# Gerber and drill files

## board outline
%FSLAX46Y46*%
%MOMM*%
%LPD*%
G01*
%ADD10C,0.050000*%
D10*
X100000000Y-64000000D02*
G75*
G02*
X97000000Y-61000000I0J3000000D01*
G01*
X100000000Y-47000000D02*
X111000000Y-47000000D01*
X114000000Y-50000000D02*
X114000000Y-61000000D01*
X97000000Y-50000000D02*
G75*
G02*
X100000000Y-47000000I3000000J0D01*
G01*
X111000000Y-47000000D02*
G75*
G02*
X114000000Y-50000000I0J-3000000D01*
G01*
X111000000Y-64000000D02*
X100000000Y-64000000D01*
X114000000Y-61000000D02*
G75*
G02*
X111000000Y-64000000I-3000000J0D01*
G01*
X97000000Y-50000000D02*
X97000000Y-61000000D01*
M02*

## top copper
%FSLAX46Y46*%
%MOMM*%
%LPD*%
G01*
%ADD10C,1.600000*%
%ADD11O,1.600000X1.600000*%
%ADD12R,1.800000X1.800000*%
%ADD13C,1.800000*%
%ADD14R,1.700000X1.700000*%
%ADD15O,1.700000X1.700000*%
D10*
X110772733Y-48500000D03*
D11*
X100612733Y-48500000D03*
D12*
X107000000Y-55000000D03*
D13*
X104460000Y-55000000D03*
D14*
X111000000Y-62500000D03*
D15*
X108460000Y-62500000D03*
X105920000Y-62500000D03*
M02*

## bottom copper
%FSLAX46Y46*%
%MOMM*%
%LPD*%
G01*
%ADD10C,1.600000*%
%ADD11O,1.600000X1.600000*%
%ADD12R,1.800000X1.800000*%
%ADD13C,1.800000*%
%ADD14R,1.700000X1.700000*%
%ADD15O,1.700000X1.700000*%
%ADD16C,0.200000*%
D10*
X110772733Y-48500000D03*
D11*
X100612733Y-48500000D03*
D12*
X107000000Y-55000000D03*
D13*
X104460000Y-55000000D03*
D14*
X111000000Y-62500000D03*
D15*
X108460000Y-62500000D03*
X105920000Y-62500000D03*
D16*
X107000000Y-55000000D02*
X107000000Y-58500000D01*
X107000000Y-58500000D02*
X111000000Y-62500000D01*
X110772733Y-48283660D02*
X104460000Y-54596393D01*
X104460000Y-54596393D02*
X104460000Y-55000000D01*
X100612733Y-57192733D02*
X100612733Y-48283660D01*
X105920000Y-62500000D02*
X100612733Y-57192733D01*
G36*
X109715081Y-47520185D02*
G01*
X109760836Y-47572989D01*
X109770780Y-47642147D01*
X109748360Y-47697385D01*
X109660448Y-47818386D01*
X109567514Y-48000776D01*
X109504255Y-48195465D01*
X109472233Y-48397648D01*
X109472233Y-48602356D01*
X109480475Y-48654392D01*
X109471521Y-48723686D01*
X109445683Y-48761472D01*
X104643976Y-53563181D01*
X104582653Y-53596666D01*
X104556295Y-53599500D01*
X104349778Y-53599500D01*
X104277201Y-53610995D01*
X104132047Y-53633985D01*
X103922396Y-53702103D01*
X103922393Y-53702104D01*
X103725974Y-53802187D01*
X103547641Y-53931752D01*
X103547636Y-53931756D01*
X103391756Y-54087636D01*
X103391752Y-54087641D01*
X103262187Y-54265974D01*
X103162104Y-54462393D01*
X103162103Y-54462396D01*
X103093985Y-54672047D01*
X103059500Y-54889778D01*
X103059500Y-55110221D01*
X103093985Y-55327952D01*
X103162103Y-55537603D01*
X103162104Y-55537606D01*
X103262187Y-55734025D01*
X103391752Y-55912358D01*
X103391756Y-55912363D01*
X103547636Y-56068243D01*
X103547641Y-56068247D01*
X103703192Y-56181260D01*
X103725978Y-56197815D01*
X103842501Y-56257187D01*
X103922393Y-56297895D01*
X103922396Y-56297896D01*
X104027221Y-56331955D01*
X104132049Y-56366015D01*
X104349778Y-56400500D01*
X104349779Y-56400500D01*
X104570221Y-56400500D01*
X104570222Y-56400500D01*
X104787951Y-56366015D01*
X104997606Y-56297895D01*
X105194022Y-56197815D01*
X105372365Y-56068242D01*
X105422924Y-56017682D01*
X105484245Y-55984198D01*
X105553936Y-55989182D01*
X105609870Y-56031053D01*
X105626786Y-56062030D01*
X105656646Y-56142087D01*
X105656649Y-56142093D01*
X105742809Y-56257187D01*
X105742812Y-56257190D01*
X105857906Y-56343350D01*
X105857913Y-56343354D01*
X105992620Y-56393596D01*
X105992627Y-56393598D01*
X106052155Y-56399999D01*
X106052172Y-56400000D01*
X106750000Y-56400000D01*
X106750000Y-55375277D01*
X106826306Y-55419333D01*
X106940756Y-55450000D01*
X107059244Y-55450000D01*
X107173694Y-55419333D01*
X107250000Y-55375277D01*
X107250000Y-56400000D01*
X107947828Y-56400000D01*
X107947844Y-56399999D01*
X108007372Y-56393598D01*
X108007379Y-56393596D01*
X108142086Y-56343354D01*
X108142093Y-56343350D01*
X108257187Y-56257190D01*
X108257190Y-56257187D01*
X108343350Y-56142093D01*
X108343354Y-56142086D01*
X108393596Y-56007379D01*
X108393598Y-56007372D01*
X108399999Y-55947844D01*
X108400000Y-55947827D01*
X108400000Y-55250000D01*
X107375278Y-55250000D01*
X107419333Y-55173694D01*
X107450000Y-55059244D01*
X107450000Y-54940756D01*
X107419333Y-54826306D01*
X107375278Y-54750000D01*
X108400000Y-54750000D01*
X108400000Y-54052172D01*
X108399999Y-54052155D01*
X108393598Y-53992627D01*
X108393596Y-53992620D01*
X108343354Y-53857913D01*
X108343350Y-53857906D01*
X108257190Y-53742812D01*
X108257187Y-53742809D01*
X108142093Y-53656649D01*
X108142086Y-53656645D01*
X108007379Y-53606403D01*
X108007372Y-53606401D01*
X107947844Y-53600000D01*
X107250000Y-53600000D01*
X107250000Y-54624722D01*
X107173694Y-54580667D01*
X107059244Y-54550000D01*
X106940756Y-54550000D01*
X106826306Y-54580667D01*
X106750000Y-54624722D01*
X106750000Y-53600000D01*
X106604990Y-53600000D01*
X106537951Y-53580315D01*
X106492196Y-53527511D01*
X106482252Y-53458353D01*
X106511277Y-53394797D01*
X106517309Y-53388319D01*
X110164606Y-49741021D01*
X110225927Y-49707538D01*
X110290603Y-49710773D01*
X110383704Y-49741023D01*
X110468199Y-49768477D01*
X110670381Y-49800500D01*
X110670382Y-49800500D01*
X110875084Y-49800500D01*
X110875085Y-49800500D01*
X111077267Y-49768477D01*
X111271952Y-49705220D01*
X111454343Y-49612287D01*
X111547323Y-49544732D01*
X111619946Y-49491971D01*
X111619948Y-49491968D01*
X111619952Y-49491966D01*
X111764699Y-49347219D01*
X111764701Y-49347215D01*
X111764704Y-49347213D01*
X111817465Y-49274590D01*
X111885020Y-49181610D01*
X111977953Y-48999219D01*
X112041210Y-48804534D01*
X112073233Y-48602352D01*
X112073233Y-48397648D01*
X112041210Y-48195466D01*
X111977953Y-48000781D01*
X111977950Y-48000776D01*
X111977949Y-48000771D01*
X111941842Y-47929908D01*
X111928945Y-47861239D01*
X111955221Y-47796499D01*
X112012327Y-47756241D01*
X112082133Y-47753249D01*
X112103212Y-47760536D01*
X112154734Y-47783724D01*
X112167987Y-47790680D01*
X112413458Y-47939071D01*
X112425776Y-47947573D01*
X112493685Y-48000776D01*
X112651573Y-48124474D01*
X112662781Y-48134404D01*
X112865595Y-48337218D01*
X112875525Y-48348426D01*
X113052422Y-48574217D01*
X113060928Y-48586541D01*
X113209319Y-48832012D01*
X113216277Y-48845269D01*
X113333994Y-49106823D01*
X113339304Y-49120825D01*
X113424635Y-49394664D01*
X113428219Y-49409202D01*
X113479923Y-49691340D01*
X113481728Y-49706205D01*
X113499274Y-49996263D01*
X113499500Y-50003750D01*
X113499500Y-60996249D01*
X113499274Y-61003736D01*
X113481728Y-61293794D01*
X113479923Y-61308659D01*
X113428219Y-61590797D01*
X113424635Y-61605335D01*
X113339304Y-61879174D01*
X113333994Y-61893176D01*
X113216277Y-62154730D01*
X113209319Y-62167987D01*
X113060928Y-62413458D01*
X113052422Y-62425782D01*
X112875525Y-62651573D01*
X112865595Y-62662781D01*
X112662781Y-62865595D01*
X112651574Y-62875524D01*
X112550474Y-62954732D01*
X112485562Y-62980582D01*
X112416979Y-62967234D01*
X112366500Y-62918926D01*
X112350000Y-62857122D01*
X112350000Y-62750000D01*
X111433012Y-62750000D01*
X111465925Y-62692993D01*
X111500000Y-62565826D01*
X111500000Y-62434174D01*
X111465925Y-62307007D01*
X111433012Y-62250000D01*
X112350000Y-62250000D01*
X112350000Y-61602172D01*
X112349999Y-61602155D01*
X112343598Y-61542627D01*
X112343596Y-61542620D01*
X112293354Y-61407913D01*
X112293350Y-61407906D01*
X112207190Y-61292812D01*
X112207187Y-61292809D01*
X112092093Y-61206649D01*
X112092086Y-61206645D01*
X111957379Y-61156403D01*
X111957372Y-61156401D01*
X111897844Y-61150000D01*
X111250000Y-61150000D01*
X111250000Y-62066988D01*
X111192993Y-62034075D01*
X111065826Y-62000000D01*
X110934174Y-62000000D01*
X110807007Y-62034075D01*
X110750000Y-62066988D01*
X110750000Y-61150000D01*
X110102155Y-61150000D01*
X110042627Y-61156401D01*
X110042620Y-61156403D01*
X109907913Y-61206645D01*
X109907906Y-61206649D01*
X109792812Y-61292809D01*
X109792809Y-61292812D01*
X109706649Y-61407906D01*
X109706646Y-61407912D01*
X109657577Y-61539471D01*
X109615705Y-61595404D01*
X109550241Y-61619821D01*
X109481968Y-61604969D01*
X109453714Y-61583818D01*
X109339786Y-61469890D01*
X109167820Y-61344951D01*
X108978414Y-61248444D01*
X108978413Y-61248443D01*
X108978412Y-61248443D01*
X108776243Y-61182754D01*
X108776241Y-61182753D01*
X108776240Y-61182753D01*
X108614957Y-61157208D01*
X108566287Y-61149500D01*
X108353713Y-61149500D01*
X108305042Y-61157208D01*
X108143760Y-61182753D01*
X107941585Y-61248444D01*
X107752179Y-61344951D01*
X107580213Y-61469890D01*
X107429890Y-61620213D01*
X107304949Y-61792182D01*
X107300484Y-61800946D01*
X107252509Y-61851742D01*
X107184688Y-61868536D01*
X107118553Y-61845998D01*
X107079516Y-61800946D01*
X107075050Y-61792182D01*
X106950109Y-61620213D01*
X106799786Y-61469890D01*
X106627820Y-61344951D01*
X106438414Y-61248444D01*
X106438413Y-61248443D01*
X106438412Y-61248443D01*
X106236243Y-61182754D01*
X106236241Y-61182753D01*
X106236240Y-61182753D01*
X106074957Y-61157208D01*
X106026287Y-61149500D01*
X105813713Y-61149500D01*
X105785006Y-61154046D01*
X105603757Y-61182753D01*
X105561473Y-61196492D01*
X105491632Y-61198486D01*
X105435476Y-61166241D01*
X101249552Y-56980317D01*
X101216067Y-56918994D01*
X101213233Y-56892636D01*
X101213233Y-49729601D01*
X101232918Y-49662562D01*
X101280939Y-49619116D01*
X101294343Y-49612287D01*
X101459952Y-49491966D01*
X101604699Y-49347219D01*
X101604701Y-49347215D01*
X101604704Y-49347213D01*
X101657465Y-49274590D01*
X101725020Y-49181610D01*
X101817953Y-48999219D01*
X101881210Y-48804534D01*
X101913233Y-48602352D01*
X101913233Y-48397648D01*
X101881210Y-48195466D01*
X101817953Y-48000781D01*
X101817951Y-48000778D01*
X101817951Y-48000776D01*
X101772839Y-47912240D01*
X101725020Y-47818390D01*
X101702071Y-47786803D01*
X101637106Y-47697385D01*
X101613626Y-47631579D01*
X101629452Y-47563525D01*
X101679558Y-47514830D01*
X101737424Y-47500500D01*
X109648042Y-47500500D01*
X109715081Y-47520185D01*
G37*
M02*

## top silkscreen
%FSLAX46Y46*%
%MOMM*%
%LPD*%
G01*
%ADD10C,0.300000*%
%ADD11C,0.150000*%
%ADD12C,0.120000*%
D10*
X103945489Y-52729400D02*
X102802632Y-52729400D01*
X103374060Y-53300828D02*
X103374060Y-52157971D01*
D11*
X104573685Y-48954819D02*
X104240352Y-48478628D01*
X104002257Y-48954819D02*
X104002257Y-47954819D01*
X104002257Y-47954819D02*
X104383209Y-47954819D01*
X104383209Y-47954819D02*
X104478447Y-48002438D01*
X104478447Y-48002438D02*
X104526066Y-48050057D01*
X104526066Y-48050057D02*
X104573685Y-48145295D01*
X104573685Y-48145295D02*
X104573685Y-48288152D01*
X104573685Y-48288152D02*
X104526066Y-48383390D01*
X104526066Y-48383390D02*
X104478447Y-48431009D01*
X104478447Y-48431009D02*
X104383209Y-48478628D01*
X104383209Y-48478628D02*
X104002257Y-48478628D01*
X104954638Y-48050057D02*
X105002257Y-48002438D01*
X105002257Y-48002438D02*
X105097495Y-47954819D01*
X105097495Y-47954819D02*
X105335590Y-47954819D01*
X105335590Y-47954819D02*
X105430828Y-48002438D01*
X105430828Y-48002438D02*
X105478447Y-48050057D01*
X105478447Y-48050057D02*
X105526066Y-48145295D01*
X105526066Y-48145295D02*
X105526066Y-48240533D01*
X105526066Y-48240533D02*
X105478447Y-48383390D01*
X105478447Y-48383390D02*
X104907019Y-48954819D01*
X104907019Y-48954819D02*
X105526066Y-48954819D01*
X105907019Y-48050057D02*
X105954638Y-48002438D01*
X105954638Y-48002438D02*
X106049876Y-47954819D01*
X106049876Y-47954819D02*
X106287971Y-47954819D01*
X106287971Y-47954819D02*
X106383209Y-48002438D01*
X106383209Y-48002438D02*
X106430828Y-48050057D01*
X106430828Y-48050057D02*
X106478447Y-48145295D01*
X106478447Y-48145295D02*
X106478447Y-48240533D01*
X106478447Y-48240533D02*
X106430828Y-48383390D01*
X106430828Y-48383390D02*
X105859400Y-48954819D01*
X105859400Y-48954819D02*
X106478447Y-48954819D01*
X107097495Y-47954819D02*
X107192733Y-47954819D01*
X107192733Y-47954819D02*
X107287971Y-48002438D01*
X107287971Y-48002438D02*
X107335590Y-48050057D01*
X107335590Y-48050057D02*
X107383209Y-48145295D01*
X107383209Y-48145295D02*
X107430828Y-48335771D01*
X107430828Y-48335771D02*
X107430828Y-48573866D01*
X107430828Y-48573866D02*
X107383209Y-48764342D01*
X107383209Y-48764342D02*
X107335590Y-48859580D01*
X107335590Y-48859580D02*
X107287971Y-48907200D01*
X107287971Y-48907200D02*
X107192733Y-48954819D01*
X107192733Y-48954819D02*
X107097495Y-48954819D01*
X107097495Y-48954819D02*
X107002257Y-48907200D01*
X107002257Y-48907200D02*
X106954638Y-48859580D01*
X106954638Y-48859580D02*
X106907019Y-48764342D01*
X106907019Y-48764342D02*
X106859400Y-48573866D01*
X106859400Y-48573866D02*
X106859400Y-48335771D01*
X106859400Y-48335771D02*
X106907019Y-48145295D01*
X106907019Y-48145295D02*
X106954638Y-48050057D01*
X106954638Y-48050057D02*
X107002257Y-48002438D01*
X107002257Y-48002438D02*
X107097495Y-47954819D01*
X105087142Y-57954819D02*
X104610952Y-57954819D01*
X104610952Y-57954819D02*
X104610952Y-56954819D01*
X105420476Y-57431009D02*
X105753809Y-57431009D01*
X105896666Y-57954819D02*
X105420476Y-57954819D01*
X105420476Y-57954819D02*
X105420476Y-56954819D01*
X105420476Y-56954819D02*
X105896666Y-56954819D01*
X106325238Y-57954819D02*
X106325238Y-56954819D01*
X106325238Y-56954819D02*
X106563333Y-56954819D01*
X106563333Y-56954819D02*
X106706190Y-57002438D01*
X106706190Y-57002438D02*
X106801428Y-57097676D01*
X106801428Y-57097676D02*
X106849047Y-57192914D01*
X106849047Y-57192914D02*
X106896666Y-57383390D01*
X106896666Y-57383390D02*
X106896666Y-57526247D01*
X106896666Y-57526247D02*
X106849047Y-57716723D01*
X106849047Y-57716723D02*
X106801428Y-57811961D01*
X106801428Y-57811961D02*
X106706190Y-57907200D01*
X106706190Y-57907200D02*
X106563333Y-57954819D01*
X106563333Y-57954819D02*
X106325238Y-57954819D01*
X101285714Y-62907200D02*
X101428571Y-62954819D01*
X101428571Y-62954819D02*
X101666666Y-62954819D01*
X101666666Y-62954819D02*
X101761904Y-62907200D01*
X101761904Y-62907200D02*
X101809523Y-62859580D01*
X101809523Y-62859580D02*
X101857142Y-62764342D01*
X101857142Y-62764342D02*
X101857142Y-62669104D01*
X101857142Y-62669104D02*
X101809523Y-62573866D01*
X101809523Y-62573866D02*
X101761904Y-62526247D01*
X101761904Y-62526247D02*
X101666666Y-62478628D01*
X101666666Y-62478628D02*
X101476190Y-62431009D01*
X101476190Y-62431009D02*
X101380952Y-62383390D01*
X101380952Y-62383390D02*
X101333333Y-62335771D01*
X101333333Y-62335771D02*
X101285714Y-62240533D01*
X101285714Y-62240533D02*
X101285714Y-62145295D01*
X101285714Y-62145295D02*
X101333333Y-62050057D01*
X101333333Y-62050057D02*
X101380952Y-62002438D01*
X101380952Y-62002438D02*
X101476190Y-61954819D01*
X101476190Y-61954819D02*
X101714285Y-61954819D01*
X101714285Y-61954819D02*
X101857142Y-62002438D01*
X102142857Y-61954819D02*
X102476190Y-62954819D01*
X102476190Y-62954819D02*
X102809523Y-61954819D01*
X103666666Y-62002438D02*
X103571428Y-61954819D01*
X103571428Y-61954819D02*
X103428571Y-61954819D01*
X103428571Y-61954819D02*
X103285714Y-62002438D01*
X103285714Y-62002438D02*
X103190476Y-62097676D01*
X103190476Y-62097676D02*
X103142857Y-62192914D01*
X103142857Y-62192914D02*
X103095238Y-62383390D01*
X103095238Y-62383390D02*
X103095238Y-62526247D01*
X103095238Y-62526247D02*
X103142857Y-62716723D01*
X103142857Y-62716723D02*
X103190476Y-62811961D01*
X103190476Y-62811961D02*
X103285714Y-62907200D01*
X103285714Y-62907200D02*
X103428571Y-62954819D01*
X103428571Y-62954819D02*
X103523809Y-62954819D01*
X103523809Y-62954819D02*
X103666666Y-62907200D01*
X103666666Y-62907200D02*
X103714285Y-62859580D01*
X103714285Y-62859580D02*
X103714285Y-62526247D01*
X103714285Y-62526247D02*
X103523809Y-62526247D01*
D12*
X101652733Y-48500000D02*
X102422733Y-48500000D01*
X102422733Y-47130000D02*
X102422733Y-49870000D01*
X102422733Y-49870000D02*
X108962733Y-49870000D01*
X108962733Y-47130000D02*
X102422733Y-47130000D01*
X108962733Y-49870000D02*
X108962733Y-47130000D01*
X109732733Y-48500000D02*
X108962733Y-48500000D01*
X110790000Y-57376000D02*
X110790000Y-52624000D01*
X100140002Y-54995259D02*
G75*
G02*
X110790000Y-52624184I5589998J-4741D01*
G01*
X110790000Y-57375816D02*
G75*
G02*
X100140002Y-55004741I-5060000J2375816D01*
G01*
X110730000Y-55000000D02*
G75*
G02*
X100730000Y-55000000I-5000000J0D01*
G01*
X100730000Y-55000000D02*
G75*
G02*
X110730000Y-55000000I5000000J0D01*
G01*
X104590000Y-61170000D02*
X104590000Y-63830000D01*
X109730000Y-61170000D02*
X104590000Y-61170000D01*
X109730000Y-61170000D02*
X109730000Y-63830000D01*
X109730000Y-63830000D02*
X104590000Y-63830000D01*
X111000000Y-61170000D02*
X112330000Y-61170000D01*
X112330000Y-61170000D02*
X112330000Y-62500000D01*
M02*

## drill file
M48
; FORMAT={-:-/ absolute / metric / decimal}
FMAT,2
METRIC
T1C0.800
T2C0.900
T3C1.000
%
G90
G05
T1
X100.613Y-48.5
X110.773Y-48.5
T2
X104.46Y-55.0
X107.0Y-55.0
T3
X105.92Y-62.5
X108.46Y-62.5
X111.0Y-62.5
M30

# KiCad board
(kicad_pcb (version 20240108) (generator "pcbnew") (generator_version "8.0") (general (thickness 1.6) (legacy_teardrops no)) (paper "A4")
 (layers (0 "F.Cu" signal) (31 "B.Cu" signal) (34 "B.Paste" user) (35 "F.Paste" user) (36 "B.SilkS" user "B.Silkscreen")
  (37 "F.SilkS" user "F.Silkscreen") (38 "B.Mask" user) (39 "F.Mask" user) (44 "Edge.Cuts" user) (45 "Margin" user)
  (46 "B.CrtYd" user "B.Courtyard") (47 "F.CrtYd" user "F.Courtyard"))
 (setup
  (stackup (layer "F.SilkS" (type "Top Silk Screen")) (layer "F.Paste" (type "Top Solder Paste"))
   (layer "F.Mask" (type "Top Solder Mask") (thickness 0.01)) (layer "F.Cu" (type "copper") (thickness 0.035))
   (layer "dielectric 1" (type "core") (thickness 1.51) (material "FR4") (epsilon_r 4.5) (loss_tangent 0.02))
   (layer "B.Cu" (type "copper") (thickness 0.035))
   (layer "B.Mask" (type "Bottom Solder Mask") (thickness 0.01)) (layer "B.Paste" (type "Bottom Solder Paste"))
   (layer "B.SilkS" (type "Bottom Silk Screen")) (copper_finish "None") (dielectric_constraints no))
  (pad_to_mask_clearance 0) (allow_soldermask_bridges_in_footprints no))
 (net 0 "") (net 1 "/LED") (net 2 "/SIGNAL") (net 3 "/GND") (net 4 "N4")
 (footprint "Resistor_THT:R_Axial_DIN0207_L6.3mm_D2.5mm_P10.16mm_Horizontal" (layer "F.Cu") (at 110.772733 48.5 180)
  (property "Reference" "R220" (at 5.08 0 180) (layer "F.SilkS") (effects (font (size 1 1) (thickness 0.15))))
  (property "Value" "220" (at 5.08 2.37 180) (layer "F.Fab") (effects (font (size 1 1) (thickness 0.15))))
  (fp_line (start 9.12 0) (end 8.35 0) (stroke (width 0.12) (type solid)) (layer "F.SilkS"))
  (fp_line (start 8.35 1.37) (end 8.35 -1.37) (stroke (width 0.12) (type solid)) (layer "F.SilkS"))
  (fp_line (start 8.35 -1.37) (end 1.81 -1.37) (stroke (width 0.12) (type solid)) (layer "F.SilkS"))
  (fp_line (start 1.81 1.37) (end 8.35 1.37) (stroke (width 0.12) (type solid)) (layer "F.SilkS"))
  (fp_line (start 1.81 -1.37) (end 1.81 1.37) (stroke (width 0.12) (type solid)) (layer "F.SilkS"))
  (fp_line (start 1.04 0) (end 1.81 0) (stroke (width 0.12) (type solid)) (layer "F.SilkS"))
  (pad "1" thru_hole circle (at 0 0 180) (size 1.6 1.6) (drill 0.8) (layers "*.Cu" "*.Mask") (remove_unused_layers no) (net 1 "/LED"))
  (pad "2" thru_hole oval (at 10.16 0 180) (size 1.6 1.6) (drill 0.8) (layers "*.Cu" "*.Mask") (remove_unused_layers no) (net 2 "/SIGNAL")))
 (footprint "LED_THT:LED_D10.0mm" (layer "F.Cu") (at 107 55 180)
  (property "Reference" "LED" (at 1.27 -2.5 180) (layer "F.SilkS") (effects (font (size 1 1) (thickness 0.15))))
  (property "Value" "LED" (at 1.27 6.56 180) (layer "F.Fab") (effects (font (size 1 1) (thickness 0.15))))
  (fp_line (start -3.79 -2.376) (end -3.79 2.376) (stroke (width 0.12) (type solid)) (layer "F.SilkS"))
  (fp_arc (start 6.859998 0.004741) (mid 2.484794 5.456407) (end -3.79 2.375816) (stroke (width 0.12) (type solid)) (layer "F.SilkS"))
  (fp_arc (start -3.79 -2.375816) (mid 2.484794 -5.456407) (end 6.859998 -0.004741) (stroke (width 0.12) (type solid)) (layer "F.SilkS"))
  (fp_circle (center 1.27 0) (end 6.27 0) (stroke (width 0.12) (type solid)) (fill none) (layer "F.SilkS"))
  (pad "1" thru_hole rect (at 0 0 180) (size 1.8 1.8) (drill 0.9) (layers "*.Cu" "*.Mask") (remove_unused_layers no) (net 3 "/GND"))
  (pad "2" thru_hole circle (at 2.54 0 180) (size 1.8 1.8) (drill 0.9) (layers "*.Cu" "*.Mask") (remove_unused_layers no) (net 1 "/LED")))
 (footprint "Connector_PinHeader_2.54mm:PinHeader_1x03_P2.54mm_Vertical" (layer "F.Cu") (at 111 62.5 -90)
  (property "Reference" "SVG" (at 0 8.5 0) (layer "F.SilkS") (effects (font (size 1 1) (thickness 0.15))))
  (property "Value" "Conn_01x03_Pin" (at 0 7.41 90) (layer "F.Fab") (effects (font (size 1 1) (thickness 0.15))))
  (fp_line (start -1.33 6.41) (end 1.33 6.41) (stroke (width 0.12) (type solid)) (layer "F.SilkS"))
  (fp_line (start -1.33 1.27) (end -1.33 6.41) (stroke (width 0.12) (type solid)) (layer "F.SilkS"))
  (fp_line (start -1.33 1.27) (end 1.33 1.27) (stroke (width 0.12) (type solid)) (layer "F.SilkS"))
  (fp_line (start 1.33 1.27) (end 1.33 6.41) (stroke (width 0.12) (type solid)) (layer "F.SilkS"))
  (fp_line (start -1.33 0) (end -1.33 -1.33) (stroke (width 0.12) (type solid)) (layer "F.SilkS"))
  (fp_line (start -1.33 -1.33) (end 0 -1.33) (stroke (width 0.12) (type solid)) (layer "F.SilkS"))
  (pad "1" thru_hole rect (at 0 0 270) (size 1.7 1.7) (drill 1) (layers "*.Cu" "*.Mask") (remove_unused_layers no) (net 3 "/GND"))
  (pad "2" thru_hole oval (at 0 2.54 270) (size 1.7 1.7) (drill 1) (layers "*.Cu" "*.Mask") (remove_unused_layers no) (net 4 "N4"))
  (pad "3" thru_hole oval (at 0 5.08 270) (size 1.7 1.7) (drill 1) (layers "*.Cu" "*.Mask") (remove_unused_layers no) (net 2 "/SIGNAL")))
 (gr_arc (start 100 64) (mid 97.87868 63.12132) (end 97 61) (locked yes) (stroke (width 0.05) (type default)) (layer "Edge.Cuts"))
 (gr_line (start 100 47) (end 111 47) (locked yes) (stroke (width 0.05) (type default)) (layer "Edge.Cuts"))
 (gr_line (start 114 50) (end 114 61) (locked yes) (stroke (width 0.05) (type default)) (layer "Edge.Cuts"))
 (gr_arc (start 97 50) (mid 97.87868 47.87868) (end 100 47) (locked yes) (stroke (width 0.05) (type default)) (layer "Edge.Cuts"))
 (gr_arc (start 111 47) (mid 113.12132 47.87868) (end 114 50) (locked yes) (stroke (width 0.05) (type default)) (layer "Edge.Cuts"))
 (gr_line (start 111 64) (end 100 64) (locked yes) (stroke (width 0.05) (type default)) (layer "Edge.Cuts"))
 (gr_arc (start 114 61) (mid 113.12132 63.12132) (end 111 64) (locked yes) (stroke (width 0.05) (type default)) (layer "Edge.Cuts"))
 (gr_line (start 97 50) (end 97 61) (locked yes) (stroke (width 0.05) (type default)) (layer "Edge.Cuts"))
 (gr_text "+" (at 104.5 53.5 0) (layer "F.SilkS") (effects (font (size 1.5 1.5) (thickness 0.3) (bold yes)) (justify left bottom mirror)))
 (segment (start 107 55) (end 107 58.5) (width 0.2) (layer "B.Cu") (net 3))
 (segment (start 107 58.5) (end 111 62.5) (width 0.2) (layer "B.Cu") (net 3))
 (segment (start 110.772733 48.28366) (end 104.46 54.596393) (width 0.2) (layer "B.Cu") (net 1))
 (segment (start 104.46 54.596393) (end 104.46 55) (width 0.2) (layer "B.Cu") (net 1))
 (segment (start 100.612733 57.192733) (end 100.612733 48.28366) (width 0.2) (layer "B.Cu") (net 2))
 (segment (start 105.92 62.5) (end 100.612733 57.192733) (width 0.2) (layer "B.Cu") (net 2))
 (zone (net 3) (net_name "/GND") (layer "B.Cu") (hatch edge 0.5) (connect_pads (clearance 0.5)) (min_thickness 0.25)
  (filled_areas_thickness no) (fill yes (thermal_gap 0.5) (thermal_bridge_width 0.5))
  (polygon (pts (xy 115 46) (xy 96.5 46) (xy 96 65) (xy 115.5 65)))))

